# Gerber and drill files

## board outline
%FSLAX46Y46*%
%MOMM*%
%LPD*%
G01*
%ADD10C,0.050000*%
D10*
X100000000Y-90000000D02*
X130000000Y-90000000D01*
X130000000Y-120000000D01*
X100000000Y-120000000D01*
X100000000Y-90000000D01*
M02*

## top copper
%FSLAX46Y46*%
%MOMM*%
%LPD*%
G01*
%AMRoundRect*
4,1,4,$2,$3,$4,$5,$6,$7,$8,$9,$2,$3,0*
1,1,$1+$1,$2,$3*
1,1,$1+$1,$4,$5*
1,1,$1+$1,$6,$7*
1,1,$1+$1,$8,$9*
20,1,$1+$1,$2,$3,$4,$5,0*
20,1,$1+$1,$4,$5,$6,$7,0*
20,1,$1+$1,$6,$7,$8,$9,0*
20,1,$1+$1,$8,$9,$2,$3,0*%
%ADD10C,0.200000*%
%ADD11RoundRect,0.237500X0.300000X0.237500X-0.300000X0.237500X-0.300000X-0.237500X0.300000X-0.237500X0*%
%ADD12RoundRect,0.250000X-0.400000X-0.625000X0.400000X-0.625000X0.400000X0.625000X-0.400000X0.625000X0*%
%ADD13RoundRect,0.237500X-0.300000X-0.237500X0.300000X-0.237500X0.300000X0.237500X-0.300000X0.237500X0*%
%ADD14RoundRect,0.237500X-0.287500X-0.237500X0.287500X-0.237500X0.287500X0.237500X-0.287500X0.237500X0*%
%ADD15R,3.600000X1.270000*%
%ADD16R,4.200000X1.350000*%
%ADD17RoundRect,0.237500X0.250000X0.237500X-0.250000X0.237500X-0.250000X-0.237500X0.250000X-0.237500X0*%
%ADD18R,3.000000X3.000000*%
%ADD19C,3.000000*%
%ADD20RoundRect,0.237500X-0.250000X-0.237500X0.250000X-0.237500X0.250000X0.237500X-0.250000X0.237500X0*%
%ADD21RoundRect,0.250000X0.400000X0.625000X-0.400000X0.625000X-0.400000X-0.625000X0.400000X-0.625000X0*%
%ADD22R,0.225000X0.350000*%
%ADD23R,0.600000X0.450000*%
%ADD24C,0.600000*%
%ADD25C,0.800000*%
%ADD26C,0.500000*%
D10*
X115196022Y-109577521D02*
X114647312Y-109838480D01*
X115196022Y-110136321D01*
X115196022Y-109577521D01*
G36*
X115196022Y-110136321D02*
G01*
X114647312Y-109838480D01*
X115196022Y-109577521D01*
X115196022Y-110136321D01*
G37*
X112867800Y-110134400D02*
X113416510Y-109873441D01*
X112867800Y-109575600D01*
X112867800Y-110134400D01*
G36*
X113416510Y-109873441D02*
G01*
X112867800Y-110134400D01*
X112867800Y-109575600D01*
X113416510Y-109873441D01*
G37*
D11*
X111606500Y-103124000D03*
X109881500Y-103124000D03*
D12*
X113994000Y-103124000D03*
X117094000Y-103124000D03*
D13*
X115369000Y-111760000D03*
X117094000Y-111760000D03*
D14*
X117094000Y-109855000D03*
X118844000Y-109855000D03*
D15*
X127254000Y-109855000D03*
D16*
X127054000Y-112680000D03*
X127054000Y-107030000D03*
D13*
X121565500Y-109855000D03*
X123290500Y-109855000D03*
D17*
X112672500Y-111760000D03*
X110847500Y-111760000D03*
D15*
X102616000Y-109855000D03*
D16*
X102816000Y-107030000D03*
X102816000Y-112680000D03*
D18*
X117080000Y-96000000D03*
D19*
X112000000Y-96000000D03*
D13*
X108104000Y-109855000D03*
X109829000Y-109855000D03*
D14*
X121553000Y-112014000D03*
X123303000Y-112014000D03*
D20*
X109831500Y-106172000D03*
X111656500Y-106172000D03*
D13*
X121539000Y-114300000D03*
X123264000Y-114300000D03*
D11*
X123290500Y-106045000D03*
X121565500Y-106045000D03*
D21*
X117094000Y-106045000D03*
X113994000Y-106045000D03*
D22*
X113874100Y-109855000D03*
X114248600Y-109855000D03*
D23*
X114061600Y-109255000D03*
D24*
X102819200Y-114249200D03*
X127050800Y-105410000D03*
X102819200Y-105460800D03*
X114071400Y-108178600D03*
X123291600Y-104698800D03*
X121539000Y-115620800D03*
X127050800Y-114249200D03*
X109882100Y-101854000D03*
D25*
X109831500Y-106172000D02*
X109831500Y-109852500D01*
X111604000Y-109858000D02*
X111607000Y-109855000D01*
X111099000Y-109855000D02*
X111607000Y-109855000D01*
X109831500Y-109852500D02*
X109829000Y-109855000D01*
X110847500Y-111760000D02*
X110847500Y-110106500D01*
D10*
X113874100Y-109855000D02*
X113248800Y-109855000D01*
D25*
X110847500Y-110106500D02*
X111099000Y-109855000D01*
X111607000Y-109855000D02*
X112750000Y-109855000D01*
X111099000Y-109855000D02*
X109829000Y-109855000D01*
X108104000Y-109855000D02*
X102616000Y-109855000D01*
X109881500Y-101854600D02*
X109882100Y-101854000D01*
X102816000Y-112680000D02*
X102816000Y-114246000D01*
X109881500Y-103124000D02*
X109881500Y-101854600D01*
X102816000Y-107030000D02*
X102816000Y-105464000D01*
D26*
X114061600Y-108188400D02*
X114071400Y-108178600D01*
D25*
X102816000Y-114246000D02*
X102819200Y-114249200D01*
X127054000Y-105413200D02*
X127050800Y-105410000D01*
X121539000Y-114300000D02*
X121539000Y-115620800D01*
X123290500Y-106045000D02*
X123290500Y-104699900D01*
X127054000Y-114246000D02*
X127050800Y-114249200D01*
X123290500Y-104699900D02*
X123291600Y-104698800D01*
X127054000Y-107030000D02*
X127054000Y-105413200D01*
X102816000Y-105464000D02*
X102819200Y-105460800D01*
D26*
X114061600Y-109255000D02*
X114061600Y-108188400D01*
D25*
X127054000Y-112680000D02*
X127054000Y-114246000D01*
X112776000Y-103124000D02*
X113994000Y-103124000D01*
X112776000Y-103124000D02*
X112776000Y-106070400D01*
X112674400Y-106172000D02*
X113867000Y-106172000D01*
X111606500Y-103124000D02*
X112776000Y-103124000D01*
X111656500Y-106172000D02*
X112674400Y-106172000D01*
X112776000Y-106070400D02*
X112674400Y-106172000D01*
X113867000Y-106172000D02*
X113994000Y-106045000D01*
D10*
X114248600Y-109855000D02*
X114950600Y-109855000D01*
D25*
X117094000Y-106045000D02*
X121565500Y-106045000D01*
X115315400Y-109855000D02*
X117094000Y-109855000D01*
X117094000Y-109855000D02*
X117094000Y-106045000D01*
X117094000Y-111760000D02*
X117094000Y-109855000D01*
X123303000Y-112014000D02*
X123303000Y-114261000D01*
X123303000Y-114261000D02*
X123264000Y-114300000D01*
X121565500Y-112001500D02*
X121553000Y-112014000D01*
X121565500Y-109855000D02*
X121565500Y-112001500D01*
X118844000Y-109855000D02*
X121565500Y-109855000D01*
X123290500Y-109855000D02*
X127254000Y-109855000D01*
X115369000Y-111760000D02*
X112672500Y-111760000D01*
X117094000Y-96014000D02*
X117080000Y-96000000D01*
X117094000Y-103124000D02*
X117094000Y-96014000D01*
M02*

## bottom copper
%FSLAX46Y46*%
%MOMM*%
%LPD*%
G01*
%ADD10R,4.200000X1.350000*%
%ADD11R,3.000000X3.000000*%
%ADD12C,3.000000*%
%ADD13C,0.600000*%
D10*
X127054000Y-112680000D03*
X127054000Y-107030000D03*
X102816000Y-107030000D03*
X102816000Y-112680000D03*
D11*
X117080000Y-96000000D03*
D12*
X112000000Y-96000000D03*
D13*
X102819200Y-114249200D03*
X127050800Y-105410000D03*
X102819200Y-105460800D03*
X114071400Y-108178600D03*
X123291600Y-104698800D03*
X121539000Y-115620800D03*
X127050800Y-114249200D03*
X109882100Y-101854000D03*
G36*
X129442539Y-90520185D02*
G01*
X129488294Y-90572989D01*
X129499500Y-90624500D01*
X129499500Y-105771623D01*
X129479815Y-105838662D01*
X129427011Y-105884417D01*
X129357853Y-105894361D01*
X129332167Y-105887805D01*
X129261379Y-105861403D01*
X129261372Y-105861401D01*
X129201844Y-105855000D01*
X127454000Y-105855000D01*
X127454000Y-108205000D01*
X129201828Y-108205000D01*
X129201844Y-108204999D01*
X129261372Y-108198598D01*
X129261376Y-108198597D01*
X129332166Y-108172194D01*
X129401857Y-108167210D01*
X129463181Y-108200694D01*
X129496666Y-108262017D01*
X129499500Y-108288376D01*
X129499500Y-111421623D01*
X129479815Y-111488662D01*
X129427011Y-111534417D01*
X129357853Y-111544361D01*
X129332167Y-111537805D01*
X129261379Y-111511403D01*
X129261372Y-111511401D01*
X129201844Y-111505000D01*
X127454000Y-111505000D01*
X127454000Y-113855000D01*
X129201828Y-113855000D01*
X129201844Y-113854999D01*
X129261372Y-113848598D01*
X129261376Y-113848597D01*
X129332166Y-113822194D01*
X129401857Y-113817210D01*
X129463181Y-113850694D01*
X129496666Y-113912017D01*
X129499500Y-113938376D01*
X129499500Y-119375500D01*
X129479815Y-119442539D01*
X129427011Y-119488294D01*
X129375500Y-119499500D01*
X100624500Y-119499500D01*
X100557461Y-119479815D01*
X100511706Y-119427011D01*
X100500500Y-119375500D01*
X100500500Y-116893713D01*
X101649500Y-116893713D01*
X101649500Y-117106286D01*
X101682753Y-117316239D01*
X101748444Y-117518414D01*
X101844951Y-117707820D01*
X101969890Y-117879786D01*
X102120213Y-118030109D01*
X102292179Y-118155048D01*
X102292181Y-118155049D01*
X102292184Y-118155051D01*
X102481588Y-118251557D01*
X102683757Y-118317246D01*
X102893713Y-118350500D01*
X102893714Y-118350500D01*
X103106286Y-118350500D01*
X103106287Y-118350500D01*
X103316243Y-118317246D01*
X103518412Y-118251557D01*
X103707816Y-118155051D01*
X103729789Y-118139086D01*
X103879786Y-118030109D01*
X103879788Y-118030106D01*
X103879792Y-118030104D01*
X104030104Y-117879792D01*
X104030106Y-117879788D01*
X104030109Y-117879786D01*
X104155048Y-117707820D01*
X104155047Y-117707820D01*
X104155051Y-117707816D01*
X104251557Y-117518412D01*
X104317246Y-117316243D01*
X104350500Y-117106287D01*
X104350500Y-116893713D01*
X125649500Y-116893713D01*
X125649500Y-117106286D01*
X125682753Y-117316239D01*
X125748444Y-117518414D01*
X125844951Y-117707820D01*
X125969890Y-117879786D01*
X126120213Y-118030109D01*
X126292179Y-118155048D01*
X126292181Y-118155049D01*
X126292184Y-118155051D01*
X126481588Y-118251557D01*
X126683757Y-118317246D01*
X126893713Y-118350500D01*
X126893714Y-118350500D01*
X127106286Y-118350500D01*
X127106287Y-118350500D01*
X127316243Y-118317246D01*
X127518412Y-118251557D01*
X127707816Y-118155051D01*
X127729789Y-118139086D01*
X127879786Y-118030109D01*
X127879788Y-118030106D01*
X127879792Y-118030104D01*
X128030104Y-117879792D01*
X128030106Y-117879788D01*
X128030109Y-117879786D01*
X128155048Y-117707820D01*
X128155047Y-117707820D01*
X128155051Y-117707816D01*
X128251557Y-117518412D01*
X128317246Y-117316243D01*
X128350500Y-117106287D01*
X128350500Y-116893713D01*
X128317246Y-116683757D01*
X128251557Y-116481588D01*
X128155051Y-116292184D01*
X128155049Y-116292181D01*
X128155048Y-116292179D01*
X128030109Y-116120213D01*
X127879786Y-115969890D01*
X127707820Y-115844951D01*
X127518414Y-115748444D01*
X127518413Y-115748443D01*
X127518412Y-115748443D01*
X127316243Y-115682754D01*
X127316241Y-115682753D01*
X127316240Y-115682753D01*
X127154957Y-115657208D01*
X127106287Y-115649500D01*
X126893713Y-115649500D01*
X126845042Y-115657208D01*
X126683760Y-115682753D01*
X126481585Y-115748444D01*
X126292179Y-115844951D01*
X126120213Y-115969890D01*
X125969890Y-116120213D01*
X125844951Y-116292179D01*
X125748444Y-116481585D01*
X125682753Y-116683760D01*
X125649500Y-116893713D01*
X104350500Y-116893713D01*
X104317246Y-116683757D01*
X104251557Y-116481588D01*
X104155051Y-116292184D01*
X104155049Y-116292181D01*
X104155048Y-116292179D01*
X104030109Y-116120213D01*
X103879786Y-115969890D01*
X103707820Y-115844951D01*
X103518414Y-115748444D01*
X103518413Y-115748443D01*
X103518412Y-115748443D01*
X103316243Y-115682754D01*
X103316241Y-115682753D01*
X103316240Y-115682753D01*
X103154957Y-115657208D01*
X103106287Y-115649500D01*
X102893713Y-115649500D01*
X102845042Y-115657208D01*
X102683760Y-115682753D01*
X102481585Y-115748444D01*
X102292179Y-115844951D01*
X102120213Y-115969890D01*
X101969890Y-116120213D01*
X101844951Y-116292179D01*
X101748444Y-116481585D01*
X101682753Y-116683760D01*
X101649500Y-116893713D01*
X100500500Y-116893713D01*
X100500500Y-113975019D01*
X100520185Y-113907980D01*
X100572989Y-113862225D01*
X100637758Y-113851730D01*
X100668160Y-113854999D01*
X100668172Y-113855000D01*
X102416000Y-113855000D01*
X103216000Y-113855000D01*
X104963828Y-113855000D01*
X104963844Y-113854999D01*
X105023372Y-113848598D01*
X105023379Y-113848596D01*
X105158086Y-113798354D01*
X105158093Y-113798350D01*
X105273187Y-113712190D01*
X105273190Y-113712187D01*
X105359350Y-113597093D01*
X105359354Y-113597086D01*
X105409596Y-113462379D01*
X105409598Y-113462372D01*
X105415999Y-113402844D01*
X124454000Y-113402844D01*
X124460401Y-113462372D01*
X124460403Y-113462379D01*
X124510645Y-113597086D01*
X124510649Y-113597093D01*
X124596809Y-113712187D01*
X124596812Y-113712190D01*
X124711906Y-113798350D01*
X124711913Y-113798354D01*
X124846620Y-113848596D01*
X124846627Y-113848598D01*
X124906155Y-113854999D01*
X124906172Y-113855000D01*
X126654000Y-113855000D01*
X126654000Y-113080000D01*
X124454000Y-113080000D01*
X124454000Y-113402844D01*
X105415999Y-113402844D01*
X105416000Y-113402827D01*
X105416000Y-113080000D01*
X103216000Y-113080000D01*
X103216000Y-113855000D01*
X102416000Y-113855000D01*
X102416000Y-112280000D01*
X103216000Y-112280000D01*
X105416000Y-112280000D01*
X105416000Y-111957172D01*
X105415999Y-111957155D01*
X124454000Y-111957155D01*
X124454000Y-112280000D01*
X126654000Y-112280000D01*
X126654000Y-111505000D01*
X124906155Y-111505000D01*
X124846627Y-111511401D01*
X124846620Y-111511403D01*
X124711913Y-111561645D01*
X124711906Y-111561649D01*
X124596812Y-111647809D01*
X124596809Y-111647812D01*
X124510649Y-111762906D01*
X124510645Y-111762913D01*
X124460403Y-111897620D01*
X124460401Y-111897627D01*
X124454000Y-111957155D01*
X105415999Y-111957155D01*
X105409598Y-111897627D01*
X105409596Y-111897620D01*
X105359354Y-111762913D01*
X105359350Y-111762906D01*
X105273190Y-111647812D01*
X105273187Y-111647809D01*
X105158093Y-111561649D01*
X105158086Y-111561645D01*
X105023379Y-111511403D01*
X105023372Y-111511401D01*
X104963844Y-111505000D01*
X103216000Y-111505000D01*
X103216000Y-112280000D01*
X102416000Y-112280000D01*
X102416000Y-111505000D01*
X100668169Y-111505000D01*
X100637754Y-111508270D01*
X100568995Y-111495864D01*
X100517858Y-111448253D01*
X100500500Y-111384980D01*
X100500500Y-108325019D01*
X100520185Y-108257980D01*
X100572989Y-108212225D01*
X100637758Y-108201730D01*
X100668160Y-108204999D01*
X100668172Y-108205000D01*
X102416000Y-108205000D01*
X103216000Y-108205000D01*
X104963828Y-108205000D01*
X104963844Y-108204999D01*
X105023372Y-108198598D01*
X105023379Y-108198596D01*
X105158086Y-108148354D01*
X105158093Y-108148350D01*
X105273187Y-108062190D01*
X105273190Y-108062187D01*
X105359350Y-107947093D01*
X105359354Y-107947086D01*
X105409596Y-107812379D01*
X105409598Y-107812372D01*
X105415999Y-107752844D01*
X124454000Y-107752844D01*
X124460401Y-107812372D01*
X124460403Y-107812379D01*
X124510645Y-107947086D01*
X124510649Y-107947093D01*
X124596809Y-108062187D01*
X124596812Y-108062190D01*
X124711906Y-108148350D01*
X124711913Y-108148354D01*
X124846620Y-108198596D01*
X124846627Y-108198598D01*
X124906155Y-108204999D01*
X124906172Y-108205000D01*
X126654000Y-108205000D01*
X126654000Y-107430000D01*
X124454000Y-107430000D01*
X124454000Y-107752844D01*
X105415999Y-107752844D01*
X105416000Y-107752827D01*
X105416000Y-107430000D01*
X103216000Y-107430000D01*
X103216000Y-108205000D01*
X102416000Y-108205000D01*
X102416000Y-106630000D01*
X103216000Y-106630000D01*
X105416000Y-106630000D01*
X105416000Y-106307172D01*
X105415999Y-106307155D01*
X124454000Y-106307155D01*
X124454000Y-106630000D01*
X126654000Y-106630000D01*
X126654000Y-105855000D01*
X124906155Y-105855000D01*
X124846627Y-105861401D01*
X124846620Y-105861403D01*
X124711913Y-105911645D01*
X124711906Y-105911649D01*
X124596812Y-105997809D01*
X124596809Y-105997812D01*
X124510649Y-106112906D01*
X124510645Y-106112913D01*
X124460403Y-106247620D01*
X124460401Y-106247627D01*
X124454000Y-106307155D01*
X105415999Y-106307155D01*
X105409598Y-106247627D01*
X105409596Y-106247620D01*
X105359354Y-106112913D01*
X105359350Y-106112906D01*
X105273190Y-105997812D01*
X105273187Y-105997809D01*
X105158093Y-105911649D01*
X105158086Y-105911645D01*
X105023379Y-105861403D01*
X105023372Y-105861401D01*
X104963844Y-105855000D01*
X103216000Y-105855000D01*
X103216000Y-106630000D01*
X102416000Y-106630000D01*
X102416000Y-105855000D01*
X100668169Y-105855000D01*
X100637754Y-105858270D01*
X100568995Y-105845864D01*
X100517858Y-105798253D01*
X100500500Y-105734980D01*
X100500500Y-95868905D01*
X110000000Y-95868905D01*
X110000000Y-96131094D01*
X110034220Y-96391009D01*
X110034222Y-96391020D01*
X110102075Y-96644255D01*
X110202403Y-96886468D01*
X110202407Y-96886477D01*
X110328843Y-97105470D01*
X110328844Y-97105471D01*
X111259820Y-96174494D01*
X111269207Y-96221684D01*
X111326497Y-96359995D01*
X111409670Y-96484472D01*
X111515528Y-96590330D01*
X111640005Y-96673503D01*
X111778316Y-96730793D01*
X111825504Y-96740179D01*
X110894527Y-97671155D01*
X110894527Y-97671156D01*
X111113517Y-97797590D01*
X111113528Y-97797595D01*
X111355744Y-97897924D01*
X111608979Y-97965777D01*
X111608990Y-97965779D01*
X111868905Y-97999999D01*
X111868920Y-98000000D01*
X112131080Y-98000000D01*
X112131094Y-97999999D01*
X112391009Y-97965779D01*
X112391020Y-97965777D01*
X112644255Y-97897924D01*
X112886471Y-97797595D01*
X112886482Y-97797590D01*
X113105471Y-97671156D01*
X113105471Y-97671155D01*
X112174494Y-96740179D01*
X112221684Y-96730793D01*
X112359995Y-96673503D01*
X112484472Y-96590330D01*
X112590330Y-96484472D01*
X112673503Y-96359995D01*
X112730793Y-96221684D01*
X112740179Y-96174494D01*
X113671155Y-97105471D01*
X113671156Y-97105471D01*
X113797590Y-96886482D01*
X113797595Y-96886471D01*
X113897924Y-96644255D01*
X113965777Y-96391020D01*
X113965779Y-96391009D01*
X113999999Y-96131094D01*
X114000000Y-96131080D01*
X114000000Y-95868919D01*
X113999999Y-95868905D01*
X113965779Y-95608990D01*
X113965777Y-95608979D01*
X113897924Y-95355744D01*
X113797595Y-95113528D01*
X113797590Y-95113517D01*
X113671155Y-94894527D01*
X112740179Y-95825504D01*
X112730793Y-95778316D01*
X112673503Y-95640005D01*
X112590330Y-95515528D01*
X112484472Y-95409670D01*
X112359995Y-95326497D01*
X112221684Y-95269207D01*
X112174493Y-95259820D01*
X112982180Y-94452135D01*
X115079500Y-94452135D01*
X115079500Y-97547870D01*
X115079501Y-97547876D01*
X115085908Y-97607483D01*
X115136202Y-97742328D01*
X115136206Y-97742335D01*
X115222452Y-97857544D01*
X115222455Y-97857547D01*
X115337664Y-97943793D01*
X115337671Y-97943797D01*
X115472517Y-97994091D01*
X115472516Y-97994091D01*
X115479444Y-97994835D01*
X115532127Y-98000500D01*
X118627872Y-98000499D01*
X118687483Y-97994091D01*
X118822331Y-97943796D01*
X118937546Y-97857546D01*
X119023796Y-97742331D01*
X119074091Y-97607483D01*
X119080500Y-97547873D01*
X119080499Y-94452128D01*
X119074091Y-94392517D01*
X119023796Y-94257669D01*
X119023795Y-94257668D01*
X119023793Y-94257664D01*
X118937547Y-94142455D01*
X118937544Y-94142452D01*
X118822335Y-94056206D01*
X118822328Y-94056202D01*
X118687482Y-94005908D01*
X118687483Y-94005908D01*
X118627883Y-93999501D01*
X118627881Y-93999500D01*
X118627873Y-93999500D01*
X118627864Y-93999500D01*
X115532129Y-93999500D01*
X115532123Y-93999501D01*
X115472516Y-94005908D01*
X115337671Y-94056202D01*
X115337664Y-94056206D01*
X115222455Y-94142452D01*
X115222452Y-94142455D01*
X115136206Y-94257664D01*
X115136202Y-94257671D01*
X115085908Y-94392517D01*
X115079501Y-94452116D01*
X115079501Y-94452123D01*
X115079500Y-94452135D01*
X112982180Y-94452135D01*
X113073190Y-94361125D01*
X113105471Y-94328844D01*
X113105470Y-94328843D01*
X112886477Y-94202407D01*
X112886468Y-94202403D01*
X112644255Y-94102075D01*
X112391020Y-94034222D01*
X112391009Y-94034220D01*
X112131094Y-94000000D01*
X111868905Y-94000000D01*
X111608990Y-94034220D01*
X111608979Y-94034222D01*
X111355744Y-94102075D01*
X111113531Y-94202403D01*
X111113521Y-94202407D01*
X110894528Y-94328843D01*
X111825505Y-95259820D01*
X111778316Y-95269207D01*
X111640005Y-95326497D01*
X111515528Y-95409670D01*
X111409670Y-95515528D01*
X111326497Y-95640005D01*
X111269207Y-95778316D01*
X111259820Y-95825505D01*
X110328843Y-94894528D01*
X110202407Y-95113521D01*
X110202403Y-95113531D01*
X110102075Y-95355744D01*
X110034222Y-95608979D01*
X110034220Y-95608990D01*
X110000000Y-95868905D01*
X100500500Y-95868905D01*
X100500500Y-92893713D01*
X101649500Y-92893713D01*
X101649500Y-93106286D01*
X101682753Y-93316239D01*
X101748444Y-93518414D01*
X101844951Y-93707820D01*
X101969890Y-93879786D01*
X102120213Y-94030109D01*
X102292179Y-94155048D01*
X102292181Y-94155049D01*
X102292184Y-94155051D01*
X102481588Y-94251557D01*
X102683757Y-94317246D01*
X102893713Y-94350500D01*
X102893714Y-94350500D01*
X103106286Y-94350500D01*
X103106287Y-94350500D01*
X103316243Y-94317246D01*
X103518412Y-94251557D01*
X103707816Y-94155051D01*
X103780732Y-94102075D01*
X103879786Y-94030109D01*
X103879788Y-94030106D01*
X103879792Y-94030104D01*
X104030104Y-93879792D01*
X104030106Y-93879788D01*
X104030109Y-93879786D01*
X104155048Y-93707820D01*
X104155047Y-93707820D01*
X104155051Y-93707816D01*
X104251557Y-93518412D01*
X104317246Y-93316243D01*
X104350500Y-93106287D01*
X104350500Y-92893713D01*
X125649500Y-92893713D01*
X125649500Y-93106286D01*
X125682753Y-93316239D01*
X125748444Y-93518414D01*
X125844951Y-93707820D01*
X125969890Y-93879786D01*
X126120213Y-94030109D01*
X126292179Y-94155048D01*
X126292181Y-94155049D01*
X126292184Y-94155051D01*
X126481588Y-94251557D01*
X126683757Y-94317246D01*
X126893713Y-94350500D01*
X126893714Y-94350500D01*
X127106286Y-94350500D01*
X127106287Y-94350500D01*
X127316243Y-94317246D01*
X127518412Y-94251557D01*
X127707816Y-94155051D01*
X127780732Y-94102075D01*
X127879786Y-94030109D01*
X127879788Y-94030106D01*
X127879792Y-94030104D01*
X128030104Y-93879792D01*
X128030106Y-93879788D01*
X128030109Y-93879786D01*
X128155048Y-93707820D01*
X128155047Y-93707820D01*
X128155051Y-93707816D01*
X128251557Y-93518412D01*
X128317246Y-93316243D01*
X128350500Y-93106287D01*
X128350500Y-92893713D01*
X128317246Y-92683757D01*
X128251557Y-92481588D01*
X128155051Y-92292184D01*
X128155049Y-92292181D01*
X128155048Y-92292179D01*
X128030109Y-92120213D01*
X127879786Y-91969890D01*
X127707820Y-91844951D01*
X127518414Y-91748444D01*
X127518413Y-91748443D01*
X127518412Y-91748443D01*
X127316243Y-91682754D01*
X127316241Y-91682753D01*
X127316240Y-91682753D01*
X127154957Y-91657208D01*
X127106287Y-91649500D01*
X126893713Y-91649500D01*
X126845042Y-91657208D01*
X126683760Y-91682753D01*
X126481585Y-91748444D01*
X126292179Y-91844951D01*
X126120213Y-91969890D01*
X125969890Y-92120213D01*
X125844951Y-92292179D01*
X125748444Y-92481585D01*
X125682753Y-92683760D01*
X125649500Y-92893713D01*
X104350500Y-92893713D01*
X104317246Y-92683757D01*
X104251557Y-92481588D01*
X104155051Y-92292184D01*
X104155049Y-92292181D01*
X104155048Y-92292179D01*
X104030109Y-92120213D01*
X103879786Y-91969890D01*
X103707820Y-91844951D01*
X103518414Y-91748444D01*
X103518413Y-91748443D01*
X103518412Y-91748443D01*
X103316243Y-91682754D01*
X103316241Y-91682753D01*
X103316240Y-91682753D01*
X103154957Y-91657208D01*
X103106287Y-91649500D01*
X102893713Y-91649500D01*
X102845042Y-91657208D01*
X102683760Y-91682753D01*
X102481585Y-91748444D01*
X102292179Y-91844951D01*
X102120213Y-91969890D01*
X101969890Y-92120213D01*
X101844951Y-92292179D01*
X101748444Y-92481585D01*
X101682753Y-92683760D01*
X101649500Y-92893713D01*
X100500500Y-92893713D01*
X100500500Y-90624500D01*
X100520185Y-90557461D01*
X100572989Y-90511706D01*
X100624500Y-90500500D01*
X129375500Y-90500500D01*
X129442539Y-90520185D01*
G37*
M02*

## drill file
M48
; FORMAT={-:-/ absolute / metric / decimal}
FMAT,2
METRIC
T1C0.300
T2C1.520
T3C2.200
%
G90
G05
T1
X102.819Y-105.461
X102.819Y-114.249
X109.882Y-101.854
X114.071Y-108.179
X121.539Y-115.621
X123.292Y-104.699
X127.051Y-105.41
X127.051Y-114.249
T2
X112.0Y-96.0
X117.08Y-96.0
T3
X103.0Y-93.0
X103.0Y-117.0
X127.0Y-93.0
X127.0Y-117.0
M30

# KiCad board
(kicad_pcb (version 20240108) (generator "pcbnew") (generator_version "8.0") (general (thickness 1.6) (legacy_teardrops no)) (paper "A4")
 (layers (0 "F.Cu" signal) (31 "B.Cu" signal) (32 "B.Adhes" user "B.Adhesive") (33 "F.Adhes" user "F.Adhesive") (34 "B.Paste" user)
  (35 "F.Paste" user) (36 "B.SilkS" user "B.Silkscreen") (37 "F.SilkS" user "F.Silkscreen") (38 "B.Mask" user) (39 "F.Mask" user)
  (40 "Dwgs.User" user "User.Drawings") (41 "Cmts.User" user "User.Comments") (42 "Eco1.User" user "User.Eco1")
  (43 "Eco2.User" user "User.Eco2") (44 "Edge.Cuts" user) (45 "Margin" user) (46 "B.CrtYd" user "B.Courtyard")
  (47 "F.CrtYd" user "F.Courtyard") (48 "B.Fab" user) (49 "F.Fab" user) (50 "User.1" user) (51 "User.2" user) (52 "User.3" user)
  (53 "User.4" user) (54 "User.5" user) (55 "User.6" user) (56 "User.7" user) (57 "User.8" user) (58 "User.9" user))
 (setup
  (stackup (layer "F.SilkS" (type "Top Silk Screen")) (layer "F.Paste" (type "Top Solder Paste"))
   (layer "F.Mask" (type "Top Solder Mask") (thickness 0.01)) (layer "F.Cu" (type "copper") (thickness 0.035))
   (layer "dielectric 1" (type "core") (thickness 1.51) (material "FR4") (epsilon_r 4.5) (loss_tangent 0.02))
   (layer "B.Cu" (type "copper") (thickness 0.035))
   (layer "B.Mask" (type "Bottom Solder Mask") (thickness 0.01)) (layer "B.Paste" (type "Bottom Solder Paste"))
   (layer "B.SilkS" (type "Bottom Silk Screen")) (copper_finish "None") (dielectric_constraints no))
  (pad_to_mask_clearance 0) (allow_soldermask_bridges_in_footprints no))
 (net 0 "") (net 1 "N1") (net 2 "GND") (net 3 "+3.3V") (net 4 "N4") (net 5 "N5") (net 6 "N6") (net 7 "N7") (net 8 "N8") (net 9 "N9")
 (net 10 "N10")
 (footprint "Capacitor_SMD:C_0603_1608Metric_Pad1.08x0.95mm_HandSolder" (layer "F.Cu") (at 110.744 103.124 180)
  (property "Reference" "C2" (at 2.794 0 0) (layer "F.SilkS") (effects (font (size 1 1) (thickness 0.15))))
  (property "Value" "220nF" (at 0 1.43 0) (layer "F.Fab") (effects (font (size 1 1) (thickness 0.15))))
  (pad "1" smd roundrect (at -0.8625 0 180) (size 1.075 0.95) (layers "F.Cu" "F.Paste" "F.Mask") (roundrect_rratio 0.25) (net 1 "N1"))
  (pad "2" smd roundrect (at 0.8625 0 180) (size 1.075 0.95) (layers "F.Cu" "F.Paste" "F.Mask") (roundrect_rratio 0.25) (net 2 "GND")))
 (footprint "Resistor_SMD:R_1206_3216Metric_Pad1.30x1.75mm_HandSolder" (layer "F.Cu") (at 115.544 103.124)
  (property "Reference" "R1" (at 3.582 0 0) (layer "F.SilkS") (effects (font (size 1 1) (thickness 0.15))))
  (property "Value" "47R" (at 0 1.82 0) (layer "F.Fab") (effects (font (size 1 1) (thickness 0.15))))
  (pad "1" smd roundrect (at -1.55 0) (size 1.3 1.75) (layers "F.Cu" "F.Paste" "F.Mask") (roundrect_rratio 0.192308) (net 1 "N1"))
  (pad "2" smd roundrect (at 1.55 0) (size 1.3 1.75) (layers "F.Cu" "F.Paste" "F.Mask") (roundrect_rratio 0.192308) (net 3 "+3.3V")))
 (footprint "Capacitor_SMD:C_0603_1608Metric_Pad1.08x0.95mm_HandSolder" (layer "F.Cu") (at 116.2315 111.76)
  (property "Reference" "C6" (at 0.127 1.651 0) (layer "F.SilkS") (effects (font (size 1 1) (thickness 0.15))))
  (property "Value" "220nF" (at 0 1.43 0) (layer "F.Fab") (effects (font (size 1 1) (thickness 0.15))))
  (pad "1" smd roundrect (at -0.8625 0) (size 1.075 0.95) (layers "F.Cu" "F.Paste" "F.Mask") (roundrect_rratio 0.25) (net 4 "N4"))
  (pad "2" smd roundrect (at 0.8625 0) (size 1.075 0.95) (layers "F.Cu" "F.Paste" "F.Mask") (roundrect_rratio 0.25) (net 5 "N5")))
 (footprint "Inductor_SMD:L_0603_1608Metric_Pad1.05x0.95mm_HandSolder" (layer "F.Cu") (at 117.969 109.855)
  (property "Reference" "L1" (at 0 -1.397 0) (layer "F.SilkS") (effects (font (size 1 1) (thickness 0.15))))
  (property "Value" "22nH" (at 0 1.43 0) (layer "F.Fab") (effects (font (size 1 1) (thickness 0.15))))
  (pad "1" smd roundrect (at -0.875 0) (size 1.05 0.95) (layers "F.Cu" "F.Paste" "F.Mask") (roundrect_rratio 0.25) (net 5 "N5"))
  (pad "2" smd roundrect (at 0.875 0) (size 1.05 0.95) (layers "F.Cu" "F.Paste" "F.Mask") (roundrect_rratio 0.25) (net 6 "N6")))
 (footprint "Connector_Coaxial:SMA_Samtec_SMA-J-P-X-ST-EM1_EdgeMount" (layer "F.Cu") (at 127.054 109.855 90)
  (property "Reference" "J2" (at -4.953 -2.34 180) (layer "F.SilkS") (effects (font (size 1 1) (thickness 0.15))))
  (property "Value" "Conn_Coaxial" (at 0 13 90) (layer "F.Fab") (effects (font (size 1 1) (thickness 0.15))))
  (pad "1" smd rect (at 0 0.2 90) (size 1.27 3.6) (layers "F.Cu" "F.Paste" "F.Mask") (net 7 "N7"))
  (pad "2" smd rect (at -2.825 0 90) (size 1.35 4.2) (layers "F.Cu" "F.Paste" "F.Mask") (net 2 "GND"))
  (pad "2" smd rect (at -2.825 0 90) (size 1.35 4.2) (layers "B.Cu" "B.Paste" "B.Mask") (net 2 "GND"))
  (pad "2" smd rect (at 2.825 0 90) (size 1.35 4.2) (layers "F.Cu" "F.Paste" "F.Mask") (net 2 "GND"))
  (pad "2" smd rect (at 2.825 0 90) (size 1.35 4.2) (layers "B.Cu" "B.Paste" "B.Mask") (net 2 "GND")))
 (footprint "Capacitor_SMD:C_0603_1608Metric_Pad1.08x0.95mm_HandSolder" (layer "F.Cu") (at 122.428 109.855)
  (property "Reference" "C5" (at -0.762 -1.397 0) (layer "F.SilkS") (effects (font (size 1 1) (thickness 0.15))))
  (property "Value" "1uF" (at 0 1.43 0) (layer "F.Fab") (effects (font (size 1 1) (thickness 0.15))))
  (pad "1" smd roundrect (at -0.8625 0) (size 1.075 0.95) (layers "F.Cu" "F.Paste" "F.Mask") (roundrect_rratio 0.25) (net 6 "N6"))
  (pad "2" smd roundrect (at 0.8625 0) (size 1.075 0.95) (layers "F.Cu" "F.Paste" "F.Mask") (roundrect_rratio 0.25) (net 7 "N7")))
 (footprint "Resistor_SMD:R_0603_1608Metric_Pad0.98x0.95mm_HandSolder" (layer "F.Cu") (at 111.76 111.76 180)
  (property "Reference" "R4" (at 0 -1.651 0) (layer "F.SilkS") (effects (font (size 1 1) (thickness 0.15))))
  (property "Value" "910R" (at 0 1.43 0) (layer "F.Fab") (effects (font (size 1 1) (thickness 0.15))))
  (pad "1" smd roundrect (at -0.9125 0 180) (size 0.975 0.95) (layers "F.Cu" "F.Paste" "F.Mask") (roundrect_rratio 0.25) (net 4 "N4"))
  (pad "2" smd roundrect (at 0.9125 0 180) (size 0.975 0.95) (layers "F.Cu" "F.Paste" "F.Mask") (roundrect_rratio 0.25) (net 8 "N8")))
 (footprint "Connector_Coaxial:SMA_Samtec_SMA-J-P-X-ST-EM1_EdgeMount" (layer "F.Cu") (at 102.816 109.855 -90)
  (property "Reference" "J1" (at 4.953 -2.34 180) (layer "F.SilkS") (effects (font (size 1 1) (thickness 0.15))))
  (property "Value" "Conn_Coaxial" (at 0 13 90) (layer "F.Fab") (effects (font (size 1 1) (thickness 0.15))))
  (pad "1" smd rect (at 0 0.2 270) (size 1.27 3.6) (layers "F.Cu" "F.Paste" "F.Mask") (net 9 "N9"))
  (pad "2" smd rect (at -2.825 0 270) (size 1.35 4.2) (layers "F.Cu" "F.Paste" "F.Mask") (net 2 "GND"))
  (pad "2" smd rect (at -2.825 0 270) (size 1.35 4.2) (layers "B.Cu" "B.Paste" "B.Mask") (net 2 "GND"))
  (pad "2" smd rect (at 2.825 0 270) (size 1.35 4.2) (layers "F.Cu" "F.Paste" "F.Mask") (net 2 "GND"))
  (pad "2" smd rect (at 2.825 0 270) (size 1.35 4.2) (layers "B.Cu" "B.Paste" "B.Mask") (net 2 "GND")))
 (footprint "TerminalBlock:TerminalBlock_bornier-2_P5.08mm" (layer "F.Cu") (at 117.08 96 180)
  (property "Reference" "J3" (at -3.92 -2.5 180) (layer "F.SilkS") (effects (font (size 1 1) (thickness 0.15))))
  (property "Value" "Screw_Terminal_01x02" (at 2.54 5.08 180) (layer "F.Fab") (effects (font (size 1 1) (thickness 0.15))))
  (pad "1" thru_hole rect (at 0 0 180) (size 3 3) (drill 1.52) (layers "*.Cu" "*.Mask") (remove_unused_layers no) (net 3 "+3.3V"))
  (pad "2" thru_hole circle (at 5.08 0 180) (size 3 3) (drill 1.52) (layers "*.Cu" "*.Mask") (remove_unused_layers no) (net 2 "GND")))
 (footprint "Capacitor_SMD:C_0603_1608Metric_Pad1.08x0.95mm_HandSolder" (layer "F.Cu") (at 108.9665 109.855)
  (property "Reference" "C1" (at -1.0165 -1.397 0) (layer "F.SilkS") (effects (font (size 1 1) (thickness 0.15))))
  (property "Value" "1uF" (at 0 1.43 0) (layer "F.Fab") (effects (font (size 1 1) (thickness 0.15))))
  (pad "1" smd roundrect (at -0.8625 0) (size 1.075 0.95) (layers "F.Cu" "F.Paste" "F.Mask") (roundrect_rratio 0.25) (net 9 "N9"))
  (pad "2" smd roundrect (at 0.8625 0) (size 1.075 0.95) (layers "F.Cu" "F.Paste" "F.Mask") (roundrect_rratio 0.25) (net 8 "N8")))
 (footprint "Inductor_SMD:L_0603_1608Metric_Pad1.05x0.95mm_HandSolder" (layer "F.Cu") (at 122.428 112.014)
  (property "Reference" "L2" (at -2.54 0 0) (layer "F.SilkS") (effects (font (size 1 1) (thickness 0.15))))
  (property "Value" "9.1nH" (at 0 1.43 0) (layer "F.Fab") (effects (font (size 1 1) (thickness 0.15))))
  (pad "1" smd roundrect (at -0.875 0) (size 1.05 0.95) (layers "F.Cu" "F.Paste" "F.Mask") (roundrect_rratio 0.25) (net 6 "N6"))
  (pad "2" smd roundrect (at 0.875 0) (size 1.05 0.95) (layers "F.Cu" "F.Paste" "F.Mask") (roundrect_rratio 0.25) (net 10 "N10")))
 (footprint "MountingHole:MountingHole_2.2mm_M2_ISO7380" (layer "F.Cu") (at 103 93)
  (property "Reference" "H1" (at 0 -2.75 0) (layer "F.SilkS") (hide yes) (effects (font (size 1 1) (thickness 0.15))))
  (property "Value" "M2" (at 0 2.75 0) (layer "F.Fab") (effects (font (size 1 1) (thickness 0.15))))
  (pad "" np_thru_hole circle (at 0 0) (size 2.2 2.2) (drill 2.2) (layers "*.Cu" "*.Mask")))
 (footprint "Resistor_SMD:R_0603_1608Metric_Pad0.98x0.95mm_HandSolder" (layer "F.Cu") (at 110.744 106.172)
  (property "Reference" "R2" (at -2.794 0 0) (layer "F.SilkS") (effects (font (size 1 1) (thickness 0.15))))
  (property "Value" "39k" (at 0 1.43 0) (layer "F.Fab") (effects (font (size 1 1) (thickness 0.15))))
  (pad "1" smd roundrect (at -0.9125 0) (size 0.975 0.95) (layers "F.Cu" "F.Paste" "F.Mask") (roundrect_rratio 0.25) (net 8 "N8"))
  (pad "2" smd roundrect (at 0.9125 0) (size 0.975 0.95) (layers "F.Cu" "F.Paste" "F.Mask") (roundrect_rratio 0.25) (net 1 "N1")))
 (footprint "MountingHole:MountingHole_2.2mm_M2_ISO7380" (layer "F.Cu") (at 127 93)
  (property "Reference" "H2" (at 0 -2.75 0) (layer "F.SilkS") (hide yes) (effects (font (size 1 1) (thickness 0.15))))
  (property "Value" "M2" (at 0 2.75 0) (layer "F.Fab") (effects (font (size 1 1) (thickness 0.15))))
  (pad "" np_thru_hole circle (at 0 0) (size 2.2 2.2) (drill 2.2) (layers "*.Cu" "*.Mask")))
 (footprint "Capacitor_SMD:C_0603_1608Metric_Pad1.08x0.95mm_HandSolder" (layer "F.Cu") (at 122.4015 114.3)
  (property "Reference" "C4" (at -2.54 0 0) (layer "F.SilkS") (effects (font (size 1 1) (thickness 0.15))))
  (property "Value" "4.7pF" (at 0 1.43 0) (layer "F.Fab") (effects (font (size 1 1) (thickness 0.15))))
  (pad "1" smd roundrect (at -0.8625 0) (size 1.075 0.95) (layers "F.Cu" "F.Paste" "F.Mask") (roundrect_rratio 0.25) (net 2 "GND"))
  (pad "2" smd roundrect (at 0.8625 0) (size 1.075 0.95) (layers "F.Cu" "F.Paste" "F.Mask") (roundrect_rratio 0.25) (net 10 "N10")))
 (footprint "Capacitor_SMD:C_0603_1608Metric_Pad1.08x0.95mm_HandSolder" (layer "F.Cu") (at 122.428 106.045 180)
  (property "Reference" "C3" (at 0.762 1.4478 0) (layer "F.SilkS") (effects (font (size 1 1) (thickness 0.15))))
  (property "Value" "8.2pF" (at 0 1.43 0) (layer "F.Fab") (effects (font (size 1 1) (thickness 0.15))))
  (pad "1" smd roundrect (at -0.8625 0 180) (size 1.075 0.95) (layers "F.Cu" "F.Paste" "F.Mask") (roundrect_rratio 0.25) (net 2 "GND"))
  (pad "2" smd roundrect (at 0.8625 0 180) (size 1.075 0.95) (layers "F.Cu" "F.Paste" "F.Mask") (roundrect_rratio 0.25) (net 5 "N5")))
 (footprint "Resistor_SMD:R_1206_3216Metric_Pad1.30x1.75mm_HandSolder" (layer "F.Cu") (at 115.544 106.045 180)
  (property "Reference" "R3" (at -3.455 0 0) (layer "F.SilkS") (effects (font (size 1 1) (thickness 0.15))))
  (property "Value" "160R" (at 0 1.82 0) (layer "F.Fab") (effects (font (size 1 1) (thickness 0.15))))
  (pad "1" smd roundrect (at -1.55 0 180) (size 1.3 1.75) (layers "F.Cu" "F.Paste" "F.Mask") (roundrect_rratio 0.192308) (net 5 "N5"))
  (pad "2" smd roundrect (at 1.55 0 180) (size 1.3 1.75) (layers "F.Cu" "F.Paste" "F.Mask") (roundrect_rratio 0.192308) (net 1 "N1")))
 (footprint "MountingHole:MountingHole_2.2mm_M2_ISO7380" (layer "F.Cu") (at 127 117)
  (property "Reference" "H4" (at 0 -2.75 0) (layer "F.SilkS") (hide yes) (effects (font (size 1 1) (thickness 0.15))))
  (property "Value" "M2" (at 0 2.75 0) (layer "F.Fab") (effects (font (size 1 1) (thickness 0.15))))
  (pad "" np_thru_hole circle (at 0 0) (size 2.2 2.2) (drill 2.2) (layers "*.Cu" "*.Mask")))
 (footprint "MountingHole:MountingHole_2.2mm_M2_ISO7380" (layer "F.Cu") (at 103 117)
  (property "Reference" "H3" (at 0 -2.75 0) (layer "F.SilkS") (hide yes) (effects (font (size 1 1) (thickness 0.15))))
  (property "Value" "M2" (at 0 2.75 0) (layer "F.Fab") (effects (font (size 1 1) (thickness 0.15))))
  (pad "" np_thru_hole circle (at 0 0) (size 2.2 2.2) (drill 2.2) (layers "*.Cu" "*.Mask")))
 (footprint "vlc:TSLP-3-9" (layer "F.Cu") (at 114.06135 109.555 90)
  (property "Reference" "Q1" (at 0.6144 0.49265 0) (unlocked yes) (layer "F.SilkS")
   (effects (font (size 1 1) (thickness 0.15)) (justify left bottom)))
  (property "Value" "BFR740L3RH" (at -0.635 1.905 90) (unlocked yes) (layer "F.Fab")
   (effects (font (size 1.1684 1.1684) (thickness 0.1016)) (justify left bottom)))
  (pad "1" smd rect (at -0.3 -0.18725 90) (size 0.35 0.225) (layers "F.Cu" "F.Paste") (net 8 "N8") (solder_mask_margin 0.1016)
   (clearance 0.15) (thermal_bridge_angle 0))
  (pad "2" smd rect (at -0.3 0.18725 90) (size 0.35 0.225) (layers "F.Cu" "F.Paste") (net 5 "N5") (solder_mask_margin 0.1016)
   (clearance 0.15) (thermal_bridge_angle 0))
  (pad "3" smd rect (at 0.3 0.00025 90) (size 0.45 0.6) (layers "F.Cu" "F.Paste") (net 2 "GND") (solder_mask_margin 0.1016)
   (thermal_bridge_angle 0)))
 (gr_poly
  (pts (xy 115.196022 109.577521) (xy 114.647312 109.83848) (xy 115.196022 110.136321)) (stroke (width 0.2) (type solid)) (fill solid)
  (layer "F.Cu") (net 5))
 (gr_poly
  (pts (xy 112.8678 110.1344) (xy 113.41651 109.873441) (xy 112.8678 109.5756)) (stroke (width 0.2) (type solid)) (fill solid)
  (layer "F.Cu") (net 8))
 (gr_rect (start 100 90) (end 130 120) (stroke (width 0.05) (type default)) (fill none) (layer "Edge.Cuts"))
 (segment (start 109.8315 106.172) (end 109.8315 109.8525) (width 0.8) (layer "F.Cu") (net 8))
 (segment (start 111.604 109.858) (end 111.607 109.855) (width 0.8) (layer "F.Cu") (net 8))
 (segment (start 111.099 109.855) (end 111.607 109.855) (width 0.8) (layer "F.Cu") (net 8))
 (segment (start 109.8315 109.8525) (end 109.829 109.855) (width 0.8) (layer "F.Cu") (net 8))
 (segment (start 110.8475 111.76) (end 110.8475 110.1065) (width 0.8) (layer "F.Cu") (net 8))
 (segment (start 113.8741 109.855) (end 113.2488 109.855) (width 0.2) (layer "F.Cu") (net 8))
 (segment (start 110.8475 110.1065) (end 111.099 109.855) (width 0.8) (layer "F.Cu") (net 8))
 (segment (start 111.607 109.855) (end 112.75 109.855) (width 0.8) (layer "F.Cu") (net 8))
 (segment (start 111.099 109.855) (end 109.829 109.855) (width 0.8) (layer "F.Cu") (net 8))
 (segment (start 108.104 109.855) (end 102.616 109.855) (width 0.8) (layer "F.Cu") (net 9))
 (segment (start 109.8815 101.8546) (end 109.8821 101.854) (width 0.8) (layer "F.Cu") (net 2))
 (segment (start 102.816 112.68) (end 102.816 114.246) (width 0.8) (layer "F.Cu") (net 2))
 (segment (start 109.8815 103.124) (end 109.8815 101.8546) (width 0.8) (layer "F.Cu") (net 2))
 (segment (start 102.816 107.03) (end 102.816 105.464) (width 0.8) (layer "F.Cu") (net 2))
 (segment (start 114.0616 108.1884) (end 114.0714 108.1786) (width 0.5) (layer "F.Cu") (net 2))
 (segment (start 102.816 114.246) (end 102.8192 114.2492) (width 0.8) (layer "F.Cu") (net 2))
 (segment (start 127.054 105.4132) (end 127.0508 105.41) (width 0.8) (layer "F.Cu") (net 2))
 (segment (start 121.539 114.3) (end 121.539 115.6208) (width 0.8) (layer "F.Cu") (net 2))
 (segment (start 123.2905 106.045) (end 123.2905 104.6999) (width 0.8) (layer "F.Cu") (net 2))
 (segment (start 127.054 114.246) (end 127.0508 114.2492) (width 0.8) (layer "F.Cu") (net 2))
 (segment (start 123.2905 104.6999) (end 123.2916 104.6988) (width 0.8) (layer "F.Cu") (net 2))
 (segment (start 127.054 107.03) (end 127.054 105.4132) (width 0.8) (layer "F.Cu") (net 2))
 (segment (start 102.816 105.464) (end 102.8192 105.4608) (width 0.8) (layer "F.Cu") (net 2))
 (segment (start 114.0616 109.255) (end 114.0616 108.1884) (width 0.5) (layer "F.Cu") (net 2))
 (segment (start 127.054 112.68) (end 127.054 114.246) (width 0.8) (layer "F.Cu") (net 2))
 (via (at 102.8192 114.2492) (size 0.6) (drill 0.3) (layers "F.Cu" "B.Cu") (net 2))
 (via (at 127.0508 105.41) (size 0.6) (drill 0.3) (layers "F.Cu" "B.Cu") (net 2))
 (via (at 102.8192 105.4608) (size 0.6) (drill 0.3) (layers "F.Cu" "B.Cu") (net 2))
 (via (at 114.0714 108.1786) (size 0.6) (drill 0.3) (layers "F.Cu" "B.Cu") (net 2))
 (via (at 123.2916 104.6988) (size 0.6) (drill 0.3) (layers "F.Cu" "B.Cu") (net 2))
 (via (at 121.539 115.6208) (size 0.6) (drill 0.3) (layers "F.Cu" "B.Cu") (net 2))
 (via (at 127.0508 114.2492) (size 0.6) (drill 0.3) (layers "F.Cu" "B.Cu") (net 2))
 (via (at 109.8821 101.854) (size 0.6) (drill 0.3) (layers "F.Cu" "B.Cu") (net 2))
 (segment (start 112.776 103.124) (end 113.994 103.124) (width 0.8) (layer "F.Cu") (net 1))
 (segment (start 112.776 103.124) (end 112.776 106.0704) (width 0.8) (layer "F.Cu") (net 1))
 (segment (start 112.6744 106.172) (end 113.867 106.172) (width 0.8) (layer "F.Cu") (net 1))
 (segment (start 111.6065 103.124) (end 112.776 103.124) (width 0.8) (layer "F.Cu") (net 1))
 (segment (start 111.6565 106.172) (end 112.6744 106.172) (width 0.8) (layer "F.Cu") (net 1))
 (segment (start 112.776 106.0704) (end 112.6744 106.172) (width 0.8) (layer "F.Cu") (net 1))
 (segment (start 113.867 106.172) (end 113.994 106.045) (width 0.8) (layer "F.Cu") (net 1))
 (segment (start 114.2486 109.855) (end 114.9506 109.855) (width 0.2) (layer "F.Cu") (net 5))
 (segment (start 117.094 106.045) (end 121.5655 106.045) (width 0.8) (layer "F.Cu") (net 5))
 (segment (start 115.3154 109.855) (end 117.094 109.855) (width 0.8) (layer "F.Cu") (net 5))
 (segment (start 117.094 109.855) (end 117.094 106.045) (width 0.8) (layer "F.Cu") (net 5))
 (segment (start 117.094 111.76) (end 117.094 109.855) (width 0.8) (layer "F.Cu") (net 5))
 (segment (start 123.303 112.014) (end 123.303 114.261) (width 0.8) (layer "F.Cu") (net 10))
 (segment (start 123.303 114.261) (end 123.264 114.3) (width 0.8) (layer "F.Cu") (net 10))
 (segment (start 121.5655 112.0015) (end 121.553 112.014) (width 0.8) (layer "F.Cu") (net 6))
 (segment (start 121.5655 109.855) (end 121.5655 112.0015) (width 0.8) (layer "F.Cu") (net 6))
 (segment (start 118.844 109.855) (end 121.5655 109.855) (width 0.8) (layer "F.Cu") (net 6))
 (segment (start 123.2905 109.855) (end 127.254 109.855) (width 0.8) (layer "F.Cu") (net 7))
 (segment (start 115.369 111.76) (end 112.6725 111.76) (width 0.8) (layer "F.Cu") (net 4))
 (segment (start 117.094 96.014) (end 117.08 96) (width 0.8) (layer "F.Cu") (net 3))
 (segment (start 117.094 103.124) (end 117.094 96.014) (width 0.8) (layer "F.Cu") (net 3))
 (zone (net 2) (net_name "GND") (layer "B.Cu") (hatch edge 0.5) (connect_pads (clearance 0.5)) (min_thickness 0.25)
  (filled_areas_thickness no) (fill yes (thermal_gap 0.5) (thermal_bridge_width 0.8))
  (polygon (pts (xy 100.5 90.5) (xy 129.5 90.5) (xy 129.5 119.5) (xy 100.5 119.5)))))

